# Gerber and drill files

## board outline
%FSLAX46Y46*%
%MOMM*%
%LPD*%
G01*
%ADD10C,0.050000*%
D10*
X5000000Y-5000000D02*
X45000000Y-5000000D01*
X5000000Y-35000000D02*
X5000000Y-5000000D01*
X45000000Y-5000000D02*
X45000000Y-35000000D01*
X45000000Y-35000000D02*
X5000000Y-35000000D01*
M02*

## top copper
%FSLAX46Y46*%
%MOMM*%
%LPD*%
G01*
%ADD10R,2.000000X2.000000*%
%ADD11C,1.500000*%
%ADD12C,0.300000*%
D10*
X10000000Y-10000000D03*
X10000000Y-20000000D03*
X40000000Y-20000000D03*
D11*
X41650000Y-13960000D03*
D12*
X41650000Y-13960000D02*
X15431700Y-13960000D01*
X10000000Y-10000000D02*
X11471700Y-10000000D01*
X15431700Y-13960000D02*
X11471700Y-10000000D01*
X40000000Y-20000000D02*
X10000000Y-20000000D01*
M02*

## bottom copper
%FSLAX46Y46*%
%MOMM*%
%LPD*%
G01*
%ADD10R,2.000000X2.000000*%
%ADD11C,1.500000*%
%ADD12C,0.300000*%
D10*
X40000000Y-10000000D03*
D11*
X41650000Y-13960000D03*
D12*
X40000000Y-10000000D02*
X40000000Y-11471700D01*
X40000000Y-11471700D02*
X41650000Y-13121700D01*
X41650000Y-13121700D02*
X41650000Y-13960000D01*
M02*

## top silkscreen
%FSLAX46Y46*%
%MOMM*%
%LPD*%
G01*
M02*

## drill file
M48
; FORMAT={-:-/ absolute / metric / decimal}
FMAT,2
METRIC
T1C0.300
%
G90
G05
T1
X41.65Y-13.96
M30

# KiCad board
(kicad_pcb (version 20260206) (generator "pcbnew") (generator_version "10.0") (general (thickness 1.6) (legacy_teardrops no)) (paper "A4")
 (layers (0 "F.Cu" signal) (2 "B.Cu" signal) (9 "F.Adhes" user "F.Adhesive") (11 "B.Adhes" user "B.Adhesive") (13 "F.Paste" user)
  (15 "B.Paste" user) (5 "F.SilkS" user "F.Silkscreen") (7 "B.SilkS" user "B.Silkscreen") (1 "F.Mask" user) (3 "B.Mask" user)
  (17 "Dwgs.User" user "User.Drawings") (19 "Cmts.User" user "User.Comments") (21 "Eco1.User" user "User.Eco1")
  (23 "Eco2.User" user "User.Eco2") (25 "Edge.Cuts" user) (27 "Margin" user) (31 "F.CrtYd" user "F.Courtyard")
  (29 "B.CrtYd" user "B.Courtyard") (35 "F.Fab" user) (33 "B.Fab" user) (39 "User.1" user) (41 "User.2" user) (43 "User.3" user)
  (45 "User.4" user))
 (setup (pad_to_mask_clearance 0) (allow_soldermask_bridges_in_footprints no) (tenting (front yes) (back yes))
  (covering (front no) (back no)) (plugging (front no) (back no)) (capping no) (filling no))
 (gr_line (start 5 5) (end 45 5) (stroke (width 0.05) (type default)) (layer "Edge.Cuts"))
 (gr_line (start 5 35) (end 5 5) (stroke (width 0.05) (type default)) (layer "Edge.Cuts"))
 (gr_line (start 45 5) (end 45 35) (stroke (width 0.05) (type default)) (layer "Edge.Cuts"))
 (gr_line (start 45 35) (end 5 35) (stroke (width 0.05) (type default)) (layer "Edge.Cuts"))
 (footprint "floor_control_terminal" (layer "F.Cu") (at 10 10)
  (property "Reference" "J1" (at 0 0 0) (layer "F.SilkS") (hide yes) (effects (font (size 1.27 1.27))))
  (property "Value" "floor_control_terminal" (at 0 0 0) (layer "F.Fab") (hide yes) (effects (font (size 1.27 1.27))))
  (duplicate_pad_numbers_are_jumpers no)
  (pad "1" smd rect (at 0 0) (size 2 2) (layers "F.Cu" "F.Paste" "F.Mask") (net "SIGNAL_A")))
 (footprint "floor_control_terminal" (layer "B.Cu") (at 40 10)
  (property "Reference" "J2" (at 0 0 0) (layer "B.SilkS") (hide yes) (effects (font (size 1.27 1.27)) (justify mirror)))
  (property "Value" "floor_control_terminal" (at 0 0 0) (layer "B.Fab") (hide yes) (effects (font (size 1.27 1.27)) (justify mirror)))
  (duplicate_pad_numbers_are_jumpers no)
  (pad "1" smd rect (at 0 0) (size 2 2) (layers "B.Cu" "B.Paste" "B.Mask") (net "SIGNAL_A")))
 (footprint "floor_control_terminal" (layer "F.Cu") (at 10 20)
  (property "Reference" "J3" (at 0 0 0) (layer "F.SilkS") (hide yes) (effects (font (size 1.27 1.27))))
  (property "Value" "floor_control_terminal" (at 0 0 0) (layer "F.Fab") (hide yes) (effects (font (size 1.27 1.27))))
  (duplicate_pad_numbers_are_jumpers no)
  (pad "1" smd rect (at 0 0) (size 2 2) (layers "F.Cu" "F.Paste" "F.Mask") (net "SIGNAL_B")))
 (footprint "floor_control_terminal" (layer "F.Cu") (at 40 20)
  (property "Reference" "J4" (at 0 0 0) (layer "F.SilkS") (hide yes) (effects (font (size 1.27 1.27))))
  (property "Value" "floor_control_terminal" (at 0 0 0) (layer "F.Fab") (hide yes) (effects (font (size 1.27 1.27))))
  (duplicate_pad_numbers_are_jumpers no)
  (pad "1" smd rect (at 0 0) (size 2 2) (layers "F.Cu" "F.Paste" "F.Mask") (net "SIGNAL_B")))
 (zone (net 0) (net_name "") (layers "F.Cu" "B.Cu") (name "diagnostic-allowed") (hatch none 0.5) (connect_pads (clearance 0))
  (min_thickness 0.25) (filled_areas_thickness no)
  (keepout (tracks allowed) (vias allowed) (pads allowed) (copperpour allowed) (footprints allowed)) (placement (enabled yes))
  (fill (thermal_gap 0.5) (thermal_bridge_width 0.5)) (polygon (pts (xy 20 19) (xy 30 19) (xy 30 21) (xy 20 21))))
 (segment (start 41.65 13.96) (end 15.4317 13.96) (width 0.3) (layer "F.Cu") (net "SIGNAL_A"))
 (segment (start 10 10) (end 11.4717 10) (width 0.3) (layer "F.Cu") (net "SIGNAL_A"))
 (segment (start 15.4317 13.96) (end 11.4717 10) (width 0.3) (layer "F.Cu") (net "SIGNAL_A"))
 (via (at 41.65 13.96) (size 1.5) (drill 0.3) (layers "F.Cu" "B.Cu") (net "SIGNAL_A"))
 (segment (start 40 10) (end 40 11.4717) (width 0.3) (layer "B.Cu") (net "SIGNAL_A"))
 (segment (start 40 11.4717) (end 41.65 13.1217) (width 0.3) (layer "B.Cu") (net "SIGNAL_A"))
 (segment (start 41.65 13.1217) (end 41.65 13.96) (width 0.3) (layer "B.Cu") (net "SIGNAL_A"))
 (segment (start 40 20) (end 10 20) (width 0.3) (layer "F.Cu") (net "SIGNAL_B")))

